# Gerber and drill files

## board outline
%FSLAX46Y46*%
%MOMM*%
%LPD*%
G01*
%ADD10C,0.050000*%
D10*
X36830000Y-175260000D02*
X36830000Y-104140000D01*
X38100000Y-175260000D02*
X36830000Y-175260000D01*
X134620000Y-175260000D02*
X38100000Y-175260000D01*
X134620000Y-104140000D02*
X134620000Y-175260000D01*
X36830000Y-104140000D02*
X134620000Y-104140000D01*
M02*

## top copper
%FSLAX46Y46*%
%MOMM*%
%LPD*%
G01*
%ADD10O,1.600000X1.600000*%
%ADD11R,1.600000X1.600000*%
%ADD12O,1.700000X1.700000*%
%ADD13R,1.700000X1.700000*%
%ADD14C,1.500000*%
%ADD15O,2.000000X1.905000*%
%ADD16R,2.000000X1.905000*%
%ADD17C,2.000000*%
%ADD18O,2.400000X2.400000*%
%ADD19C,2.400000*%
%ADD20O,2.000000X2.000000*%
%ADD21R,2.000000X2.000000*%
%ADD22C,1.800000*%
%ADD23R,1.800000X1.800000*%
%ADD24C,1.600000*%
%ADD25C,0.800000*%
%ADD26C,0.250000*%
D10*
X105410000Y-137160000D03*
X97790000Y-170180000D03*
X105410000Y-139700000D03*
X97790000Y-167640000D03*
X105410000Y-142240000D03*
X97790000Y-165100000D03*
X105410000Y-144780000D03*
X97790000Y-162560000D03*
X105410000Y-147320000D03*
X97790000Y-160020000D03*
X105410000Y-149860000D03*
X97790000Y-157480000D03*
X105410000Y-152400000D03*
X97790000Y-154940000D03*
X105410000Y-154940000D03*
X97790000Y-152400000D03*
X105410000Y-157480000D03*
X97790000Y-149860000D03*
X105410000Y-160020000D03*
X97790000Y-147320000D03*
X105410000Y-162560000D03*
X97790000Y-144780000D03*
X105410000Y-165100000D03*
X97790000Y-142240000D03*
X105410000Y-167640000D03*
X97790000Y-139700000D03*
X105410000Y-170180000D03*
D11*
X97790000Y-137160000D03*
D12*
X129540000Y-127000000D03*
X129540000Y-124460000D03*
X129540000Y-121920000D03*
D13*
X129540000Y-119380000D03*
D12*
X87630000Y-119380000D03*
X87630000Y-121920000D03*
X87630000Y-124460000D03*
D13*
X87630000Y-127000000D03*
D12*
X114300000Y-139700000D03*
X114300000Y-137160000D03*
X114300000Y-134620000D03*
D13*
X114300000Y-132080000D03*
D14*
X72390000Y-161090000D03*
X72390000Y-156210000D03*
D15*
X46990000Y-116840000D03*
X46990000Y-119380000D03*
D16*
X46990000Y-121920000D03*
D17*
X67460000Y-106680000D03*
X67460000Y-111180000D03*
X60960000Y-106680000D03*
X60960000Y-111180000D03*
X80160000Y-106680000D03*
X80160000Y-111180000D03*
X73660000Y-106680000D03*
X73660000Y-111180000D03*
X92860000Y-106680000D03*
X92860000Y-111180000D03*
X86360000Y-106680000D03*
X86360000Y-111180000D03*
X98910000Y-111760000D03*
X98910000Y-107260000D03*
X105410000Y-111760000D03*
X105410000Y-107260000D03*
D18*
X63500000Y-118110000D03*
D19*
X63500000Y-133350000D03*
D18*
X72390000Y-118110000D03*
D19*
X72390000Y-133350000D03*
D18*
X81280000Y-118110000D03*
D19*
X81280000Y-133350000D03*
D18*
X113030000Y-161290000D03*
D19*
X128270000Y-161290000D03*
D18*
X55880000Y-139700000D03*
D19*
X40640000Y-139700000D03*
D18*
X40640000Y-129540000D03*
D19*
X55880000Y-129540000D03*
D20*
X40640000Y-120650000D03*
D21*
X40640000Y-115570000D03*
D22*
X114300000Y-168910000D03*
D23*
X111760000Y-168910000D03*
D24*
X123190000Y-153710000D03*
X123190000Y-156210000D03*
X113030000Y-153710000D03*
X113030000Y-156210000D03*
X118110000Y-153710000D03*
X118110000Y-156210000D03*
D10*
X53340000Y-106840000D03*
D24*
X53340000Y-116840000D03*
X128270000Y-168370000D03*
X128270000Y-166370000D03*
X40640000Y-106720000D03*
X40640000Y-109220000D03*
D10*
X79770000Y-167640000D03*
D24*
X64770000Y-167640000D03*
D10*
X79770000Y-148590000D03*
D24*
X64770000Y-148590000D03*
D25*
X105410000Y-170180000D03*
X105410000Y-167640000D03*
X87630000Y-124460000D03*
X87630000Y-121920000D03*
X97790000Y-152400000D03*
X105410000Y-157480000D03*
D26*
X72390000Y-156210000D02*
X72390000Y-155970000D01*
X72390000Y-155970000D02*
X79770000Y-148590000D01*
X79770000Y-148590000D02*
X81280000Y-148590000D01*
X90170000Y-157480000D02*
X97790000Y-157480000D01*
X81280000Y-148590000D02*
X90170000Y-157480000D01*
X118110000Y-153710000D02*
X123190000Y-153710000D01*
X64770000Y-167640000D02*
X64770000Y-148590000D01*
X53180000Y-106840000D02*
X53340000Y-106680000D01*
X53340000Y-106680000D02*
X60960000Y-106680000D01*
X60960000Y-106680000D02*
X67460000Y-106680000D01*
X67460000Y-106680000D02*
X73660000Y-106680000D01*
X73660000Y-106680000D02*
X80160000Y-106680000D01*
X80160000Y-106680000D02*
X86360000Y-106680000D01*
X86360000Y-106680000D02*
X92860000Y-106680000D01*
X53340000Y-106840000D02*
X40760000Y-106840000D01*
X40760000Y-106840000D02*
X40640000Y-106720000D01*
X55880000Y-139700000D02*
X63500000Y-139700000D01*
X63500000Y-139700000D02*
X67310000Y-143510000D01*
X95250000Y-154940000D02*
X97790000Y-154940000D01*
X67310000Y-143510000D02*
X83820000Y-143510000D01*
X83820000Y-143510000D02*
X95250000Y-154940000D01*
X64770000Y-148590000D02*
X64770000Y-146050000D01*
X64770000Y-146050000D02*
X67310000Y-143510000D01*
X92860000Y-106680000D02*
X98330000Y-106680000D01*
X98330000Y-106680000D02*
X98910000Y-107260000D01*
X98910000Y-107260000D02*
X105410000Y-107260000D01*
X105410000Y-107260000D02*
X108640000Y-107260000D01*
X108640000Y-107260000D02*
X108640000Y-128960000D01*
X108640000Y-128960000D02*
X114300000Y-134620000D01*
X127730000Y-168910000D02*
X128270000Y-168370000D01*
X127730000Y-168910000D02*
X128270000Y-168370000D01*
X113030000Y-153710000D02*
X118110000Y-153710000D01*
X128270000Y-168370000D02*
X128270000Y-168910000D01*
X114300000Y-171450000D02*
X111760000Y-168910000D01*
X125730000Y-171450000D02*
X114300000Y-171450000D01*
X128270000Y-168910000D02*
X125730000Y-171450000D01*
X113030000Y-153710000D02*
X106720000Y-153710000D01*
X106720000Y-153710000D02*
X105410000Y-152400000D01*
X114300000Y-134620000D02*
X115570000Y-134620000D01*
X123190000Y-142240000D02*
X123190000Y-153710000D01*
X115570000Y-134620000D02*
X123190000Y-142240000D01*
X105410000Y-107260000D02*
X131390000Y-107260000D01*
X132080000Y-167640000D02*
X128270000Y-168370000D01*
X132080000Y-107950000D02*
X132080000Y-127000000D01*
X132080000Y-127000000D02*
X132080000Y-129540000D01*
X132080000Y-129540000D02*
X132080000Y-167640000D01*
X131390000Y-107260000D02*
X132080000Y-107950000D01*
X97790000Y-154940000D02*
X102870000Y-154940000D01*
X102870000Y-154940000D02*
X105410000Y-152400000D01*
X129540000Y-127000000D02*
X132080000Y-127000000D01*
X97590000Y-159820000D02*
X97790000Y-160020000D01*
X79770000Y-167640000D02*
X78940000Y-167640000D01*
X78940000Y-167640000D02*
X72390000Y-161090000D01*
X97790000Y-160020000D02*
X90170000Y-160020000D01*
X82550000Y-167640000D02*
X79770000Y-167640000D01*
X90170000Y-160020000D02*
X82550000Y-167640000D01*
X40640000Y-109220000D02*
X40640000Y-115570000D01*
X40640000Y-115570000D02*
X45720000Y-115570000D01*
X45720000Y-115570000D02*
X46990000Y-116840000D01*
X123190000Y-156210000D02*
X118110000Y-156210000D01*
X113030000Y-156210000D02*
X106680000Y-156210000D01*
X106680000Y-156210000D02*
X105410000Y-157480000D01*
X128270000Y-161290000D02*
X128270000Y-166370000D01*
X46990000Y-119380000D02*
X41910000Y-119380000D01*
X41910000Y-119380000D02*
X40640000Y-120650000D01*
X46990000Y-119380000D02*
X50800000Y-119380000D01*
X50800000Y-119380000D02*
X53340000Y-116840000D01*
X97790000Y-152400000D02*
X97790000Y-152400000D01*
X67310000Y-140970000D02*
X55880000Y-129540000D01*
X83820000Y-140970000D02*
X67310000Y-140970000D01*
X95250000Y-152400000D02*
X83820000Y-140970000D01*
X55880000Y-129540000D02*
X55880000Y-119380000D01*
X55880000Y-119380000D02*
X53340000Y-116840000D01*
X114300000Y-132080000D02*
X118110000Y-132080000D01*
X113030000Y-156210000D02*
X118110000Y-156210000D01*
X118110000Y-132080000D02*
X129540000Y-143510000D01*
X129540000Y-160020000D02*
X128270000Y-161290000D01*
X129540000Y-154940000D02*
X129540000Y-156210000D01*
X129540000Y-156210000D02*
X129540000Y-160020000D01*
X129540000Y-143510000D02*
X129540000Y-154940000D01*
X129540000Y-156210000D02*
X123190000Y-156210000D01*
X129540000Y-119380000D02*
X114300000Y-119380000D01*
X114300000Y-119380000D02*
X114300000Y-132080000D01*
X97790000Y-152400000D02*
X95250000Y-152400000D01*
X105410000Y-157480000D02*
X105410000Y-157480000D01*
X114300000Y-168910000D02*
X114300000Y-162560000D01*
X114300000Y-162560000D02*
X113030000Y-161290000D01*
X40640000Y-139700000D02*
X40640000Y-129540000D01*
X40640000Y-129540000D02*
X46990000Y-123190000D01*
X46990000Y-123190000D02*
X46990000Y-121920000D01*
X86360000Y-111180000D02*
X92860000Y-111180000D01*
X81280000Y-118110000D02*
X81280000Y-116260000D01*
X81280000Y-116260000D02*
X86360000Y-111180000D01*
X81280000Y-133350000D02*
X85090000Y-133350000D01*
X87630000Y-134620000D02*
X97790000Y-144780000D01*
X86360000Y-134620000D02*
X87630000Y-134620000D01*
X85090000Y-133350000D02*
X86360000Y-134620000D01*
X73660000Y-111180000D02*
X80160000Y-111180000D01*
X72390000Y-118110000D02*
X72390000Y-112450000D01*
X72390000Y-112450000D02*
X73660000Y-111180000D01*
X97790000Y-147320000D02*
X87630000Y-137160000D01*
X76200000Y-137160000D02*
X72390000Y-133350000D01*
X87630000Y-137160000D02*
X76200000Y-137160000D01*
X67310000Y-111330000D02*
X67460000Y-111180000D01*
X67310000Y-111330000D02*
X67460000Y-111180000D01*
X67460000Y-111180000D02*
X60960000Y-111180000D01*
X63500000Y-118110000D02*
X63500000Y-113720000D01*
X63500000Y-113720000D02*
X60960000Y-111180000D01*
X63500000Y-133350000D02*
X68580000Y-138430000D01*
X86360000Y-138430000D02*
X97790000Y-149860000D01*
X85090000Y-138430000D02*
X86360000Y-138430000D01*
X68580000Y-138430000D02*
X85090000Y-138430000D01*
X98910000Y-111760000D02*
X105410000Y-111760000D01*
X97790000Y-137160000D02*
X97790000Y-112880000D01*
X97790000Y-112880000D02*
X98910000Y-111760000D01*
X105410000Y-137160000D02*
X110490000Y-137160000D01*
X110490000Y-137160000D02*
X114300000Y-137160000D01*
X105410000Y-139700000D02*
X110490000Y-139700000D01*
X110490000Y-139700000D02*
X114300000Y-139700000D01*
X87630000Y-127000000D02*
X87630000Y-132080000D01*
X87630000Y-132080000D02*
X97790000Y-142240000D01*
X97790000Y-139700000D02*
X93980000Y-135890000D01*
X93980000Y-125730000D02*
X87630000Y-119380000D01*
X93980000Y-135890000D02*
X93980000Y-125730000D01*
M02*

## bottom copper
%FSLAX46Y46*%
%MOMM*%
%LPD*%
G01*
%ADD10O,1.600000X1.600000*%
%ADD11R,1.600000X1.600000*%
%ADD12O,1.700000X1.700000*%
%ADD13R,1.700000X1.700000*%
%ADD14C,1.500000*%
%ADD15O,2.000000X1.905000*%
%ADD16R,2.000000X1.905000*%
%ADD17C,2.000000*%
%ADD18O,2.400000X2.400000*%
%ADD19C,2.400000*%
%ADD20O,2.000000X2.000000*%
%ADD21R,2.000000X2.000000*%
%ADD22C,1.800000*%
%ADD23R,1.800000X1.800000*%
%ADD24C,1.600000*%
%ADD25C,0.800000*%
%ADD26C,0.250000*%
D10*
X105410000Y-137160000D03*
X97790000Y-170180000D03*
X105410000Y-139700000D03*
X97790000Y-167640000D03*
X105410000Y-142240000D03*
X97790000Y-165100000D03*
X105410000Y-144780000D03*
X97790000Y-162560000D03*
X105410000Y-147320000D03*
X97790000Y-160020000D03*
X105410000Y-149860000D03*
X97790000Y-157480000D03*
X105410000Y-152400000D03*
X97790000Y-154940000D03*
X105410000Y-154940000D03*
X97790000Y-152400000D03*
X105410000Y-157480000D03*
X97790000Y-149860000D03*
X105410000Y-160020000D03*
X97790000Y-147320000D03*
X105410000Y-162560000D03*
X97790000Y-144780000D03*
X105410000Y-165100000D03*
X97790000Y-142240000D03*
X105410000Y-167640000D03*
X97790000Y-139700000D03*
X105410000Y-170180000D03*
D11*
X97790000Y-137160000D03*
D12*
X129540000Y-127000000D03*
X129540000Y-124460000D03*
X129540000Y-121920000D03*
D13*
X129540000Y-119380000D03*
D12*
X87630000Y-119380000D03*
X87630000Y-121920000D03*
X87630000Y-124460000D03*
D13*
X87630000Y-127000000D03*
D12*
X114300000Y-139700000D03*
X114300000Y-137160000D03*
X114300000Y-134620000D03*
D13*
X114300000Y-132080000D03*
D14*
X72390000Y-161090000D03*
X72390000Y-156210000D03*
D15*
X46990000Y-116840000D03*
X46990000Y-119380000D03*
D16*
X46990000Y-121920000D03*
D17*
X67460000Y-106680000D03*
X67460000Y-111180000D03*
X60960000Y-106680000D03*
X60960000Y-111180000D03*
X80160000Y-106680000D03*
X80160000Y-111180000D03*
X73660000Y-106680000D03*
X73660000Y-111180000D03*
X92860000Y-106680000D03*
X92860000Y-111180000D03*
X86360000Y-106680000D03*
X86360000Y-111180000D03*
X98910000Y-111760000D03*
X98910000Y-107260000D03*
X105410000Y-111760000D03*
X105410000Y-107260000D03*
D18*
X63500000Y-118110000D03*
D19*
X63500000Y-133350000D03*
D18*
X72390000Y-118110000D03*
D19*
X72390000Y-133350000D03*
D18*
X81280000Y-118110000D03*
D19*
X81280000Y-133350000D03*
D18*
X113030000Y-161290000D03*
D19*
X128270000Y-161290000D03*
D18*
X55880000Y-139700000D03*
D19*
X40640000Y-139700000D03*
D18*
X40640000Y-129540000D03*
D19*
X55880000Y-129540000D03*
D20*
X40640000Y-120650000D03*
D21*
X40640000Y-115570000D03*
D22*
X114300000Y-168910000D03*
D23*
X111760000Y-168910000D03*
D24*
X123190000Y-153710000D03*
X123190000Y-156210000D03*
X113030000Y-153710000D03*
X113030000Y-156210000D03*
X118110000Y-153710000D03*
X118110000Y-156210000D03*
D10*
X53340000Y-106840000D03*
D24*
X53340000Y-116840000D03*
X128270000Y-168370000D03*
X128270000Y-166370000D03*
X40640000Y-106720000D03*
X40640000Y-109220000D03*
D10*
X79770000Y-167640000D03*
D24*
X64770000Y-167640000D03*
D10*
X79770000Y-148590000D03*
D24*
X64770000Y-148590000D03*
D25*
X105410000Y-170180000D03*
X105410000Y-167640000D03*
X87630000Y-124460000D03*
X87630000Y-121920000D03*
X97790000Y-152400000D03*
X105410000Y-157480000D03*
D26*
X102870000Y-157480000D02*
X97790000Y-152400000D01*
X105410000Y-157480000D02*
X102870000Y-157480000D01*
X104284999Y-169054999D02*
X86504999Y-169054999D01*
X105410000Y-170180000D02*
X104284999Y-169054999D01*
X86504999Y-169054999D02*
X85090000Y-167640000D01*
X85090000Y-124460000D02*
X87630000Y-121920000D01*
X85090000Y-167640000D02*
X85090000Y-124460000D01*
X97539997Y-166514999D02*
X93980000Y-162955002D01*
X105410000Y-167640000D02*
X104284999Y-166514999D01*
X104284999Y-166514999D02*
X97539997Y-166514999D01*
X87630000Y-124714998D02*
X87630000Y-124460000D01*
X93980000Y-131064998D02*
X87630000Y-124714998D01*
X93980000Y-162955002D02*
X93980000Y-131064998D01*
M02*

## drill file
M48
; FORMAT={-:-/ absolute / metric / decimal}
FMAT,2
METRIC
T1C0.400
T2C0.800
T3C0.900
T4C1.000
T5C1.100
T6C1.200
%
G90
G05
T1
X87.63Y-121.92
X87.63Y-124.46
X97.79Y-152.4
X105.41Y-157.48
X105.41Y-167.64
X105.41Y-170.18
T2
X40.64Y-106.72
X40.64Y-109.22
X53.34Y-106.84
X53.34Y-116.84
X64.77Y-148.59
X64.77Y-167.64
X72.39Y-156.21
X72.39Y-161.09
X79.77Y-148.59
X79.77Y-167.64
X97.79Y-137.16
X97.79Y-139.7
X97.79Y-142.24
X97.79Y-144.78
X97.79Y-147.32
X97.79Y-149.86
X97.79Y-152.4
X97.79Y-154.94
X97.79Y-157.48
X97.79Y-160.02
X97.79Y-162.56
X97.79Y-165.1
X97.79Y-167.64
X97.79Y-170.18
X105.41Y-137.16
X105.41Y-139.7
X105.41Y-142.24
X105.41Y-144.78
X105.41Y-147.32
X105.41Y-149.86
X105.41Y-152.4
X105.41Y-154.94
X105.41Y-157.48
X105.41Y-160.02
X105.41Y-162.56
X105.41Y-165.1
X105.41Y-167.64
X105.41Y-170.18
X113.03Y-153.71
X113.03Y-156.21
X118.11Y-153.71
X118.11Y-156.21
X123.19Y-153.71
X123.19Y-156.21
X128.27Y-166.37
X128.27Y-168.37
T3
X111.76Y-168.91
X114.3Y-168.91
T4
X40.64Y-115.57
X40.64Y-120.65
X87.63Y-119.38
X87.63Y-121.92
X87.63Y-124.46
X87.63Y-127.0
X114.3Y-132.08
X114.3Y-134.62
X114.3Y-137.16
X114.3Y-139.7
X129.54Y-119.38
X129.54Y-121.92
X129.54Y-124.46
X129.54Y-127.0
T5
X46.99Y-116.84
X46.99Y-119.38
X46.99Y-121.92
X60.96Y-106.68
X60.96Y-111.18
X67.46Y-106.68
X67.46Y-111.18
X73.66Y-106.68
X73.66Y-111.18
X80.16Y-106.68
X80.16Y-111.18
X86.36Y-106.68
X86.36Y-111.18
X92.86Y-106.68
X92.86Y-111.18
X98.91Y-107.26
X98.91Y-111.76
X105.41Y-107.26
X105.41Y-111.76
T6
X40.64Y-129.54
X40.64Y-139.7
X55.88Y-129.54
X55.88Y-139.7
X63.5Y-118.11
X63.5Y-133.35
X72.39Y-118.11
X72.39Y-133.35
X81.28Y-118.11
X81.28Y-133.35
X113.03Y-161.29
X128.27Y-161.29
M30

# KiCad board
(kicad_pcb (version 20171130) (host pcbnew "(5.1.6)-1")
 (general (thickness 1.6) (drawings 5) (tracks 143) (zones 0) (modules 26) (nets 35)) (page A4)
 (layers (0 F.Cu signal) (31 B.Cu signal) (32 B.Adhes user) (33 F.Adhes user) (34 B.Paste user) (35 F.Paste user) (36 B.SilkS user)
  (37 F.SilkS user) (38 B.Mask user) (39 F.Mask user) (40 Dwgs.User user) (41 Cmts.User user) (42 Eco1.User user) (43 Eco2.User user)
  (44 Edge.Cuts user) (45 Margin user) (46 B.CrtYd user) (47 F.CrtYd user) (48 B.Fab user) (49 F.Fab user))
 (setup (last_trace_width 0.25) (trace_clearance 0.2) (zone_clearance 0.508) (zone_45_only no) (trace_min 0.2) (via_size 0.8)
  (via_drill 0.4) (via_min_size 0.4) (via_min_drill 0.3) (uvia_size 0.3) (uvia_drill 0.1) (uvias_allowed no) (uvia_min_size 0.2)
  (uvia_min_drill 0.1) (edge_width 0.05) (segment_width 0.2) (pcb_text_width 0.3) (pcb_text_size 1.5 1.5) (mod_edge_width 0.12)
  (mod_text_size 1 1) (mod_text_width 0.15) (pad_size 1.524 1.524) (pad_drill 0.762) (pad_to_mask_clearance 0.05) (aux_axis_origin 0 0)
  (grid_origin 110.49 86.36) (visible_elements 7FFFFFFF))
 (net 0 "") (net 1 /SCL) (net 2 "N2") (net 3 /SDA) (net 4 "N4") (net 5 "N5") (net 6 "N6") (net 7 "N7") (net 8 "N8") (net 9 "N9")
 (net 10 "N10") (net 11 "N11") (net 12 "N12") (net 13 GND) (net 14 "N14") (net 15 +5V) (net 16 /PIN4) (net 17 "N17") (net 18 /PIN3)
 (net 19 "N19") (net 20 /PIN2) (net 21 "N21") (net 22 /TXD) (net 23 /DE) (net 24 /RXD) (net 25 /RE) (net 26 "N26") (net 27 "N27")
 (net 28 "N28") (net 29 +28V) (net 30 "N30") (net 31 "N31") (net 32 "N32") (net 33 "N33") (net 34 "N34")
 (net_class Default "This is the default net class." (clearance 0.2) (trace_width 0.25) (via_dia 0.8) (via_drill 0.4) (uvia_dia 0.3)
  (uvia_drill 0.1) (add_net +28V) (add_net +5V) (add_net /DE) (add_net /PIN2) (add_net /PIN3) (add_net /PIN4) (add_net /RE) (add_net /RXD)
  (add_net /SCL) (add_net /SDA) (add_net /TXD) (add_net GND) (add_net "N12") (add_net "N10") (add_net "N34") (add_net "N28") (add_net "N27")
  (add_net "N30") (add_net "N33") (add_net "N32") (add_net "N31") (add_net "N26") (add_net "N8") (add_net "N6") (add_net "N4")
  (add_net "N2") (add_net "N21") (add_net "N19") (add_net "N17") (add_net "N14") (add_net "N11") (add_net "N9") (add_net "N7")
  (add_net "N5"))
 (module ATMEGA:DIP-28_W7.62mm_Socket (layer F.Cu) (at 97.79 137.16)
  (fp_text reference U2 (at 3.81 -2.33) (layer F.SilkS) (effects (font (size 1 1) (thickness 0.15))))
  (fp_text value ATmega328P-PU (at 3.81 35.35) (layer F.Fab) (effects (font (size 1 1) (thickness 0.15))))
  (pad 28 thru_hole oval (at 7.62 0) (size 1.6 1.6) (drill 0.8) (layers *.Cu *.Mask) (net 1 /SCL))
  (pad 14 thru_hole oval (at 0 33.02) (size 1.6 1.6) (drill 0.8) (layers *.Cu *.Mask) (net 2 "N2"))
  (pad 27 thru_hole oval (at 7.62 2.54) (size 1.6 1.6) (drill 0.8) (layers *.Cu *.Mask) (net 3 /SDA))
  (pad 13 thru_hole oval (at 0 30.48) (size 1.6 1.6) (drill 0.8) (layers *.Cu *.Mask) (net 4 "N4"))
  (pad 26 thru_hole oval (at 7.62 5.08) (size 1.6 1.6) (drill 0.8) (layers *.Cu *.Mask) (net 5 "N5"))
  (pad 12 thru_hole oval (at 0 27.94) (size 1.6 1.6) (drill 0.8) (layers *.Cu *.Mask) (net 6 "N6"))
  (pad 25 thru_hole oval (at 7.62 7.62) (size 1.6 1.6) (drill 0.8) (layers *.Cu *.Mask) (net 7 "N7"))
  (pad 11 thru_hole oval (at 0 25.4) (size 1.6 1.6) (drill 0.8) (layers *.Cu *.Mask) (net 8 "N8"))
  (pad 24 thru_hole oval (at 7.62 10.16) (size 1.6 1.6) (drill 0.8) (layers *.Cu *.Mask) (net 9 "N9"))
  (pad 10 thru_hole oval (at 0 22.86) (size 1.6 1.6) (drill 0.8) (layers *.Cu *.Mask) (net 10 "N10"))
  (pad 23 thru_hole oval (at 7.62 12.7) (size 1.6 1.6) (drill 0.8) (layers *.Cu *.Mask) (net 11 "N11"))
  (pad 9 thru_hole oval (at 0 20.32) (size 1.6 1.6) (drill 0.8) (layers *.Cu *.Mask) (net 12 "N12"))
  (pad 22 thru_hole oval (at 7.62 15.24) (size 1.6 1.6) (drill 0.8) (layers *.Cu *.Mask) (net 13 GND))
  (pad 8 thru_hole oval (at 0 17.78) (size 1.6 1.6) (drill 0.8) (layers *.Cu *.Mask) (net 13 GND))
  (pad 21 thru_hole oval (at 7.62 17.78) (size 1.6 1.6) (drill 0.8) (layers *.Cu *.Mask) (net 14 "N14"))
  (pad 7 thru_hole oval (at 0 15.24) (size 1.6 1.6) (drill 0.8) (layers *.Cu *.Mask) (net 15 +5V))
  (pad 20 thru_hole oval (at 7.62 20.32) (size 1.6 1.6) (drill 0.8) (layers *.Cu *.Mask) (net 15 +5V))
  (pad 6 thru_hole oval (at 0 12.7) (size 1.6 1.6) (drill 0.8) (layers *.Cu *.Mask) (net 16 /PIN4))
  (pad 19 thru_hole oval (at 7.62 22.86) (size 1.6 1.6) (drill 0.8) (layers *.Cu *.Mask) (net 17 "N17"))
  (pad 5 thru_hole oval (at 0 10.16) (size 1.6 1.6) (drill 0.8) (layers *.Cu *.Mask) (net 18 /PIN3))
  (pad 18 thru_hole oval (at 7.62 25.4) (size 1.6 1.6) (drill 0.8) (layers *.Cu *.Mask) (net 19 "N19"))
  (pad 4 thru_hole oval (at 0 7.62) (size 1.6 1.6) (drill 0.8) (layers *.Cu *.Mask) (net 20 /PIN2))
  (pad 17 thru_hole oval (at 7.62 27.94) (size 1.6 1.6) (drill 0.8) (layers *.Cu *.Mask) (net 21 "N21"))
  (pad 3 thru_hole oval (at 0 5.08) (size 1.6 1.6) (drill 0.8) (layers *.Cu *.Mask) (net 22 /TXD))
  (pad 16 thru_hole oval (at 7.62 30.48) (size 1.6 1.6) (drill 0.8) (layers *.Cu *.Mask) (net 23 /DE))
  (pad 2 thru_hole oval (at 0 2.54) (size 1.6 1.6) (drill 0.8) (layers *.Cu *.Mask) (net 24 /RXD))
  (pad 15 thru_hole oval (at 7.62 33.02) (size 1.6 1.6) (drill 0.8) (layers *.Cu *.Mask) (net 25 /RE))
  (pad 1 thru_hole rect (at 0 0) (size 1.6 1.6) (drill 0.8) (layers *.Cu *.Mask) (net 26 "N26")))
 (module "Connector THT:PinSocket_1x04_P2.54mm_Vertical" (layer F.Cu) (at 129.54 119.38)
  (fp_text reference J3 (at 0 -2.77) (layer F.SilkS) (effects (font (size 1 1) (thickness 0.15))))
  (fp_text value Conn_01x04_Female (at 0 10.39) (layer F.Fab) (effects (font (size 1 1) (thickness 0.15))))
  (pad 4 thru_hole oval (at 0 7.62) (size 1.7 1.7) (drill 1) (layers *.Cu *.Mask) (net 13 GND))
  (pad 3 thru_hole oval (at 0 5.08) (size 1.7 1.7) (drill 1) (layers *.Cu *.Mask) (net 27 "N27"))
  (pad 2 thru_hole oval (at 0 2.54) (size 1.7 1.7) (drill 1) (layers *.Cu *.Mask) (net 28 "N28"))
  (pad 1 thru_hole rect (at 0 0) (size 1.7 1.7) (drill 1) (layers *.Cu *.Mask) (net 15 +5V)))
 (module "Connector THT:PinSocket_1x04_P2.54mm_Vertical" (layer F.Cu) (at 87.63 127 180)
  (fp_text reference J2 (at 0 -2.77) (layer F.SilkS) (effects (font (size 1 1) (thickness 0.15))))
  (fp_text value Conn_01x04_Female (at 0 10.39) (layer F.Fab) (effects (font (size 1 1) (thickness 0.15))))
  (pad 4 thru_hole oval (at 0 7.62 180) (size 1.7 1.7) (drill 1) (layers *.Cu *.Mask) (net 24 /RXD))
  (pad 3 thru_hole oval (at 0 5.08 180) (size 1.7 1.7) (drill 1) (layers *.Cu *.Mask) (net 25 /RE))
  (pad 2 thru_hole oval (at 0 2.54 180) (size 1.7 1.7) (drill 1) (layers *.Cu *.Mask) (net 23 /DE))
  (pad 1 thru_hole rect (at 0 0 180) (size 1.7 1.7) (drill 1) (layers *.Cu *.Mask) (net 22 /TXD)))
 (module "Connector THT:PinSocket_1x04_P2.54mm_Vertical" (layer F.Cu) (at 114.3 132.08)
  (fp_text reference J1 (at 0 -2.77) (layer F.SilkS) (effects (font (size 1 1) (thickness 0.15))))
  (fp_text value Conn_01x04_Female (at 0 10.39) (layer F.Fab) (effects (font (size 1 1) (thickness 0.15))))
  (pad 4 thru_hole oval (at 0 7.62) (size 1.7 1.7) (drill 1) (layers *.Cu *.Mask) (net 3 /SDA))
  (pad 3 thru_hole oval (at 0 5.08) (size 1.7 1.7) (drill 1) (layers *.Cu *.Mask) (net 1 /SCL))
  (pad 2 thru_hole oval (at 0 2.54) (size 1.7 1.7) (drill 1) (layers *.Cu *.Mask) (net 13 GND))
  (pad 1 thru_hole rect (at 0 0) (size 1.7 1.7) (drill 1) (layers *.Cu *.Mask) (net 15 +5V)))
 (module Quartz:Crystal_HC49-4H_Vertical (layer F.Cu) (at 72.39 156.21 270)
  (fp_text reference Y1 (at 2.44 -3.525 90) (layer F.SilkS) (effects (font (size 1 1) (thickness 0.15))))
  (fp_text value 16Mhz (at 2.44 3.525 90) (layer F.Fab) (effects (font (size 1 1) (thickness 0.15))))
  (pad 2 thru_hole circle (at 4.88 0 270) (size 1.5 1.5) (drill 0.8) (layers *.Cu *.Mask) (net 10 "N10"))
  (pad 1 thru_hole circle (at 0 0 270) (size 1.5 1.5) (drill 0.8) (layers *.Cu *.Mask) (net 12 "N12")))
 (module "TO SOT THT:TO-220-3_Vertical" (layer F.Cu) (at 46.99 121.92 90)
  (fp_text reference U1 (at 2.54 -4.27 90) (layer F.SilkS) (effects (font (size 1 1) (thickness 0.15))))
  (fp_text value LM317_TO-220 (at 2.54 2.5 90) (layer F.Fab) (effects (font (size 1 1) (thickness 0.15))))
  (pad 3 thru_hole oval (at 5.08 0 90) (size 1.905 2) (drill 1.1) (layers *.Cu *.Mask) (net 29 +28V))
  (pad 2 thru_hole oval (at 2.54 0 90) (size 1.905 2) (drill 1.1) (layers *.Cu *.Mask) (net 15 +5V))
  (pad 1 thru_hole rect (at 0 0 90) (size 1.905 2) (drill 1.1) (layers *.Cu *.Mask) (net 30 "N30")))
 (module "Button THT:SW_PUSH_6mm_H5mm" (layer F.Cu) (at 60.96 106.68)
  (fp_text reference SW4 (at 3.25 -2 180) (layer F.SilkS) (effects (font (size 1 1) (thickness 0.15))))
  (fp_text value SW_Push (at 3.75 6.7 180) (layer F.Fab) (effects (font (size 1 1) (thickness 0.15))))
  (pad 1 thru_hole circle (at 6.5 0 90) (size 2 2) (drill 1.1) (layers *.Cu *.Mask) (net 13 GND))
  (pad 2 thru_hole circle (at 6.5 4.5 90) (size 2 2) (drill 1.1) (layers *.Cu *.Mask) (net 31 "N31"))
  (pad 1 thru_hole circle (at 0 0 90) (size 2 2) (drill 1.1) (layers *.Cu *.Mask) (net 13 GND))
  (pad 2 thru_hole circle (at 0 4.5 90) (size 2 2) (drill 1.1) (layers *.Cu *.Mask) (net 31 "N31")))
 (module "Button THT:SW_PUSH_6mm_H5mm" (layer F.Cu) (at 73.66 106.68)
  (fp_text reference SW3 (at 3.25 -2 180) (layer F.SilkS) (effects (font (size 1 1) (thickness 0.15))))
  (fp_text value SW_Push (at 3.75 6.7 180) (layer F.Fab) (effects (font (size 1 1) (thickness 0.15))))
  (pad 1 thru_hole circle (at 6.5 0 90) (size 2 2) (drill 1.1) (layers *.Cu *.Mask) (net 13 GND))
  (pad 2 thru_hole circle (at 6.5 4.5 90) (size 2 2) (drill 1.1) (layers *.Cu *.Mask) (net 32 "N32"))
  (pad 1 thru_hole circle (at 0 0 90) (size 2 2) (drill 1.1) (layers *.Cu *.Mask) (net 13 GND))
  (pad 2 thru_hole circle (at 0 4.5 90) (size 2 2) (drill 1.1) (layers *.Cu *.Mask) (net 32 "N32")))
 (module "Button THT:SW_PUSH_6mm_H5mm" (layer F.Cu) (at 86.36 106.68)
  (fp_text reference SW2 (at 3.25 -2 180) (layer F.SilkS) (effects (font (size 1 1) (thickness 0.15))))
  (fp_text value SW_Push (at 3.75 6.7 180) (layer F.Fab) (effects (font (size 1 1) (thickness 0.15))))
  (pad 1 thru_hole circle (at 6.5 0 90) (size 2 2) (drill 1.1) (layers *.Cu *.Mask) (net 13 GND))
  (pad 2 thru_hole circle (at 6.5 4.5 90) (size 2 2) (drill 1.1) (layers *.Cu *.Mask) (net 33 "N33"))
  (pad 1 thru_hole circle (at 0 0 90) (size 2 2) (drill 1.1) (layers *.Cu *.Mask) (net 13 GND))
  (pad 2 thru_hole circle (at 0 4.5 90) (size 2 2) (drill 1.1) (layers *.Cu *.Mask) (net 33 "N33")))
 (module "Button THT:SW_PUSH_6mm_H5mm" (layer F.Cu) (at 105.41 111.76 180)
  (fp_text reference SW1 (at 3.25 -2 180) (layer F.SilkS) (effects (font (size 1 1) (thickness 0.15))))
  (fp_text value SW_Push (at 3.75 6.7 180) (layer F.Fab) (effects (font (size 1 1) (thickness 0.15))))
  (pad 1 thru_hole circle (at 6.5 0 270) (size 2 2) (drill 1.1) (layers *.Cu *.Mask) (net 26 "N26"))
  (pad 2 thru_hole circle (at 6.5 4.5 270) (size 2 2) (drill 1.1) (layers *.Cu *.Mask) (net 13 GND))
  (pad 1 thru_hole circle (at 0 0 270) (size 2 2) (drill 1.1) (layers *.Cu *.Mask) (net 26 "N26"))
  (pad 2 thru_hole circle (at 0 4.5 270) (size 2 2) (drill 1.1) (layers *.Cu *.Mask) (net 13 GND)))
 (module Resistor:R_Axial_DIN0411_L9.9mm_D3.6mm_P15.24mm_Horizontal (layer F.Cu) (at 63.5 133.35 90)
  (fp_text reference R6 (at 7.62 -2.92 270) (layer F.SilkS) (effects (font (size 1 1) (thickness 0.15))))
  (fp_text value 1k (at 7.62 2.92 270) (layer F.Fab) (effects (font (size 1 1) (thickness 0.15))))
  (pad 2 thru_hole oval (at 15.24 0 90) (size 2.4 2.4) (drill 1.2) (layers *.Cu *.Mask) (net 31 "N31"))
  (pad 1 thru_hole circle (at 0 0 90) (size 2.4 2.4) (drill 1.2) (layers *.Cu *.Mask) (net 16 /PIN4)))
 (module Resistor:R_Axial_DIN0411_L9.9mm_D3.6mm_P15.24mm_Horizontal (layer F.Cu) (at 72.39 133.35 90)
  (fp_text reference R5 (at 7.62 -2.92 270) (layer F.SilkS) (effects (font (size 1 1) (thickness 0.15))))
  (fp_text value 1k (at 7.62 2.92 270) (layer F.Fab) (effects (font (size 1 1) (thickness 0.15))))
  (pad 2 thru_hole oval (at 15.24 0 90) (size 2.4 2.4) (drill 1.2) (layers *.Cu *.Mask) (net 32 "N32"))
  (pad 1 thru_hole circle (at 0 0 90) (size 2.4 2.4) (drill 1.2) (layers *.Cu *.Mask) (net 18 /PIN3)))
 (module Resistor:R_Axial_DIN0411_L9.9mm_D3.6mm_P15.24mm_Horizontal (layer F.Cu) (at 81.28 133.35 90)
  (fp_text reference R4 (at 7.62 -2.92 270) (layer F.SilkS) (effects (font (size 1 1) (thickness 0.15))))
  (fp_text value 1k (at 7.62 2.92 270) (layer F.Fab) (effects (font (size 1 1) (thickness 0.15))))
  (pad 2 thru_hole oval (at 15.24 0 90) (size 2.4 2.4) (drill 1.2) (layers *.Cu *.Mask) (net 33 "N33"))
  (pad 1 thru_hole circle (at 0 0 90) (size 2.4 2.4) (drill 1.2) (layers *.Cu *.Mask) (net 20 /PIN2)))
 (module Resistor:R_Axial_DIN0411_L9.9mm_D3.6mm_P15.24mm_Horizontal (layer F.Cu) (at 128.27 161.29 180)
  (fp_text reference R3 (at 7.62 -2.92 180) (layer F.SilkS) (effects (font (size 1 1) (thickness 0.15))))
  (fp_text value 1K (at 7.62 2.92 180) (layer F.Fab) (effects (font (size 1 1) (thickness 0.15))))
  (pad 2 thru_hole oval (at 15.24 0 180) (size 2.4 2.4) (drill 1.2) (layers *.Cu *.Mask) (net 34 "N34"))
  (pad 1 thru_hole circle (at 0 0 180) (size 2.4 2.4) (drill 1.2) (layers *.Cu *.Mask) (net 15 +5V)))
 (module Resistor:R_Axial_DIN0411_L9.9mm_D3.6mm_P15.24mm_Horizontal (layer F.Cu) (at 40.64 139.7)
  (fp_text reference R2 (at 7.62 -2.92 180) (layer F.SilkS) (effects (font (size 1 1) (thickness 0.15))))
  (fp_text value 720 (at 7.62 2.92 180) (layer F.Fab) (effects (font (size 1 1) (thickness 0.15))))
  (pad 2 thru_hole oval (at 15.24 0) (size 2.4 2.4) (drill 1.2) (layers *.Cu *.Mask) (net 13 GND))
  (pad 1 thru_hole circle (at 0 0) (size 2.4 2.4) (drill 1.2) (layers *.Cu *.Mask) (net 30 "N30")))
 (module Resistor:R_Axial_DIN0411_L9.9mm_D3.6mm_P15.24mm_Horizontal (layer F.Cu) (at 55.88 129.54 180)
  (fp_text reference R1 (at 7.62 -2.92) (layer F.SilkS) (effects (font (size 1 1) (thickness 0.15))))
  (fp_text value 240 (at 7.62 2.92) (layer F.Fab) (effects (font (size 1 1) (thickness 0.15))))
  (pad 2 thru_hole oval (at 15.24 0 180) (size 2.4 2.4) (drill 1.2) (layers *.Cu *.Mask) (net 30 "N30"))
  (pad 1 thru_hole circle (at 0 0 180) (size 2.4 2.4) (drill 1.2) (layers *.Cu *.Mask) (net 15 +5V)))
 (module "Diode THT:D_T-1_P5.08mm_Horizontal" (layer F.Cu) (at 40.64 115.57 270)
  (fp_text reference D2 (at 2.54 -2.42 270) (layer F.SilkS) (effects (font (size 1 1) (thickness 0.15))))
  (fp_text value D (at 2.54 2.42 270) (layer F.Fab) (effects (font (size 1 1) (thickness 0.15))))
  (pad 2 thru_hole oval (at 5.08 0 270) (size 2 2) (drill 1) (layers *.Cu *.Mask) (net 15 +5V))
  (pad 1 thru_hole rect (at 0 0 270) (size 2 2) (drill 1) (layers *.Cu *.Mask) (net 29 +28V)))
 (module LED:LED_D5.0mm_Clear (layer F.Cu) (at 111.76 168.91)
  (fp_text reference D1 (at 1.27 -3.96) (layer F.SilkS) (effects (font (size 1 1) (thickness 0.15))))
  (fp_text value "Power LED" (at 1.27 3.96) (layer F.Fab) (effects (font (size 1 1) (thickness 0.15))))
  (pad 2 thru_hole circle (at 2.54 0) (size 1.8 1.8) (drill 0.9) (layers *.Cu *.Mask) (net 34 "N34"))
  (pad 1 thru_hole rect (at 0 0) (size 1.8 1.8) (drill 0.9) (layers *.Cu *.Mask) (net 13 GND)))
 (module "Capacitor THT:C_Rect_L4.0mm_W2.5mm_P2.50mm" (layer F.Cu) (at 123.19 156.21 90)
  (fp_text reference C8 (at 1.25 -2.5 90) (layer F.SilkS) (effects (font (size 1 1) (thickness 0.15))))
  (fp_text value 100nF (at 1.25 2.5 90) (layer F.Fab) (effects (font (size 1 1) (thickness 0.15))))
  (pad 2 thru_hole circle (at 2.5 0 90) (size 1.6 1.6) (drill 0.8) (layers *.Cu *.Mask) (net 13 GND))
  (pad 1 thru_hole circle (at 0 0 90) (size 1.6 1.6) (drill 0.8) (layers *.Cu *.Mask) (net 15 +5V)))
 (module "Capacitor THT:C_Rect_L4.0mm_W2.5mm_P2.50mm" (layer F.Cu) (at 113.03 156.21 90)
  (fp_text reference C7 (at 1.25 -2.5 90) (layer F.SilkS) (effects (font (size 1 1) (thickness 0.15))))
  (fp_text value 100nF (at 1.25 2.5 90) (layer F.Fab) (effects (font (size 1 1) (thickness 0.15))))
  (pad 2 thru_hole circle (at 2.5 0 90) (size 1.6 1.6) (drill 0.8) (layers *.Cu *.Mask) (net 13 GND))
  (pad 1 thru_hole circle (at 0 0 90) (size 1.6 1.6) (drill 0.8) (layers *.Cu *.Mask) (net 15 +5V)))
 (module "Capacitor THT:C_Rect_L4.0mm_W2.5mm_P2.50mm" (layer F.Cu) (at 118.11 156.21 90)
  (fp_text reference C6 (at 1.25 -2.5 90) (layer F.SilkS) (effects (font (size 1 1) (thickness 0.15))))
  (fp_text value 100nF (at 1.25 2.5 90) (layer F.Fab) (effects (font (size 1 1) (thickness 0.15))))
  (pad 2 thru_hole circle (at 2.5 0 90) (size 1.6 1.6) (drill 0.8) (layers *.Cu *.Mask) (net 13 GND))
  (pad 1 thru_hole circle (at 0 0 90) (size 1.6 1.6) (drill 0.8) (layers *.Cu *.Mask) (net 15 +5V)))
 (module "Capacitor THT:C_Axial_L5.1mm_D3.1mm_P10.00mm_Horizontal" (layer F.Cu) (at 53.34 116.84 90)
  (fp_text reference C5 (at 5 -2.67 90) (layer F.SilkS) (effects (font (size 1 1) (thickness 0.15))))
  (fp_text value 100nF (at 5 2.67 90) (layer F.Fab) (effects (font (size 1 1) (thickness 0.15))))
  (pad 2 thru_hole oval (at 10 0 90) (size 1.6 1.6) (drill 0.8) (layers *.Cu *.Mask) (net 13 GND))
  (pad 1 thru_hole circle (at 0 0 90) (size 1.6 1.6) (drill 0.8) (layers *.Cu *.Mask) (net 15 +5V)))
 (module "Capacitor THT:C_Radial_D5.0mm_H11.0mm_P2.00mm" (layer F.Cu) (at 128.27 166.37 270)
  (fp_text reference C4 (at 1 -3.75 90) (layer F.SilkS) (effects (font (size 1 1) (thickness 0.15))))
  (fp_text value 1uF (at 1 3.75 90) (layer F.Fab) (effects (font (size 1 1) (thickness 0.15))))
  (pad 2 thru_hole circle (at 2 0 270) (size 1.6 1.6) (drill 0.8) (layers *.Cu *.Mask) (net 13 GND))
  (pad 1 thru_hole circle (at 0 0 270) (size 1.6 1.6) (drill 0.8) (layers *.Cu *.Mask) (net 15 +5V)))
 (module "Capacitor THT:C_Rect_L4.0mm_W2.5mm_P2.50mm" (layer F.Cu) (at 40.64 109.22 90)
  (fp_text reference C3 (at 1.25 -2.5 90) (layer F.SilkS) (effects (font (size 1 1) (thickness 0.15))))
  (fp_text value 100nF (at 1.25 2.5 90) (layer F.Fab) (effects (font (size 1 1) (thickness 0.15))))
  (pad 2 thru_hole circle (at 2.5 0 90) (size 1.6 1.6) (drill 0.8) (layers *.Cu *.Mask) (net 13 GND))
  (pad 1 thru_hole circle (at 0 0 90) (size 1.6 1.6) (drill 0.8) (layers *.Cu *.Mask) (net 29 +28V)))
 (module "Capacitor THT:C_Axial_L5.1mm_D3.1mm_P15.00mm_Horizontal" (layer F.Cu) (at 64.77 167.64)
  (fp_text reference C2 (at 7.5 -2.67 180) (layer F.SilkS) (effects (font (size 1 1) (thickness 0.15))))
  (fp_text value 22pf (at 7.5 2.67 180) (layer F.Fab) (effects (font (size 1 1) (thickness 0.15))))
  (pad 2 thru_hole oval (at 15 0) (size 1.6 1.6) (drill 0.8) (layers *.Cu *.Mask) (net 10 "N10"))
  (pad 1 thru_hole circle (at 0 0) (size 1.6 1.6) (drill 0.8) (layers *.Cu *.Mask) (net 13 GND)))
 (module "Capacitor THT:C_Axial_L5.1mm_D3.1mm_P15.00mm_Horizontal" (layer F.Cu) (at 64.77 148.59)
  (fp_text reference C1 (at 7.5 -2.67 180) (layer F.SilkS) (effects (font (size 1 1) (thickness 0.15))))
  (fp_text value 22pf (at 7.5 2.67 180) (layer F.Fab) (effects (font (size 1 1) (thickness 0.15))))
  (pad 2 thru_hole oval (at 15 0) (size 1.6 1.6) (drill 0.8) (layers *.Cu *.Mask) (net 12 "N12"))
  (pad 1 thru_hole circle (at 0 0) (size 1.6 1.6) (drill 0.8) (layers *.Cu *.Mask) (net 13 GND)))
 (gr_line (start 36.83 175.26) (end 36.83 104.14) (angle 90) (layer Edge.Cuts) (width 0.05))
 (gr_line (start 38.1 175.26) (end 36.83 175.26) (angle 90) (layer Edge.Cuts) (width 0.05))
 (gr_line (start 134.62 175.26) (end 38.1 175.26) (angle 90) (layer Edge.Cuts) (width 0.05))
 (gr_line (start 134.62 104.14) (end 134.62 175.26) (angle 90) (layer Edge.Cuts) (width 0.05))
 (gr_line (start 36.83 104.14) (end 134.62 104.14) (angle 90) (layer Edge.Cuts) (width 0.05))
 (via (at 105.41 170.18) (size 0.8) (drill 0.4) (layers F.Cu B.Cu) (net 25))
 (via (at 105.41 167.64) (size 0.8) (drill 0.4) (layers F.Cu B.Cu) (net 23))
 (via (at 87.63 124.46) (size 0.8) (drill 0.4) (layers F.Cu B.Cu) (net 23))
 (via (at 87.63 121.92) (size 0.8) (drill 0.4) (layers F.Cu B.Cu) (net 25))
 (segment (start 72.39 156.21) (end 72.39 155.97) (width 0.25) (layer F.Cu) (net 12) (status C00000))
 (segment (start 72.39 155.97) (end 79.77 148.59) (width 0.25) (layer F.Cu) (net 12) (status C00000))
 (segment (start 79.77 148.59) (end 81.28 148.59) (width 0.25) (layer F.Cu) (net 12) (status 400000))
 (segment (start 90.17 157.48) (end 97.79 157.48) (width 0.25) (layer F.Cu) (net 12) (status 800000))
 (segment (start 81.28 148.59) (end 90.17 157.48) (width 0.25) (layer F.Cu) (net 12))
 (segment (start 118.11 153.71) (end 123.19 153.71) (width 0.25) (layer F.Cu) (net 13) (status C00000))
 (segment (start 64.77 167.64) (end 64.77 148.59) (width 0.25) (layer F.Cu) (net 13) (status C00000))
 (segment (start 53.18 106.84) (end 53.34 106.68) (width 0.25) (layer F.Cu) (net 13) (status C00000))
 (segment (start 53.34 106.68) (end 60.96 106.68) (width 0.25) (layer F.Cu) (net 13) (status C00000))
 (segment (start 60.96 106.68) (end 67.46 106.68) (width 0.25) (layer F.Cu) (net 13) (status C00000))
 (segment (start 67.46 106.68) (end 73.66 106.68) (width 0.25) (layer F.Cu) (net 13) (status C00000))
 (segment (start 73.66 106.68) (end 80.16 106.68) (width 0.25) (layer F.Cu) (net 13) (status C00000))
 (segment (start 80.16 106.68) (end 86.36 106.68) (width 0.25) (layer F.Cu) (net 13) (status C00000))
 (segment (start 86.36 106.68) (end 92.86 106.68) (width 0.25) (layer F.Cu) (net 13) (status C00000))
 (segment (start 53.34 106.84) (end 40.76 106.84) (width 0.25) (layer F.Cu) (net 13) (status C00000))
 (segment (start 40.76 106.84) (end 40.64 106.72) (width 0.25) (layer F.Cu) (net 13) (status C00000))
 (segment (start 55.88 139.7) (end 63.5 139.7) (width 0.25) (layer F.Cu) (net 13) (status 400000))
 (segment (start 63.5 139.7) (end 67.31 143.51) (width 0.25) (layer F.Cu) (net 13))
 (segment (start 95.25 154.94) (end 97.79 154.94) (width 0.25) (layer F.Cu) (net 13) (status 800000))
 (segment (start 67.31 143.51) (end 83.82 143.51) (width 0.25) (layer F.Cu) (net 13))
 (segment (start 83.82 143.51) (end 95.25 154.94) (width 0.25) (layer F.Cu) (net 13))
 (segment (start 64.77 148.59) (end 64.77 146.05) (width 0.25) (layer F.Cu) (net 13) (status 400000))
 (segment (start 64.77 146.05) (end 67.31 143.51) (width 0.25) (layer F.Cu) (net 13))
 (segment (start 92.86 106.68) (end 98.33 106.68) (width 0.25) (layer F.Cu) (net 13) (status C00000))
 (segment (start 98.33 106.68) (end 98.91 107.26) (width 0.25) (layer F.Cu) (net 13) (status C00000))
 (segment (start 98.91 107.26) (end 105.41 107.26) (width 0.25) (layer F.Cu) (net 13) (status C00000))
 (segment (start 105.41 107.26) (end 108.64 107.26) (width 0.25) (layer F.Cu) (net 13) (status 400000))
 (segment (start 108.64 107.26) (end 108.64 128.96) (width 0.25) (layer F.Cu) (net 13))
 (segment (start 108.64 128.96) (end 114.3 134.62) (width 0.25) (layer F.Cu) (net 13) (status 800000))
 (segment (start 127.73 168.91) (end 128.27 168.37) (width 0.25) (layer F.Cu) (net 13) (status C00000))
 (segment (start 127.73 168.91) (end 128.27 168.37) (width 0.25) (layer F.Cu) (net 13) (status C00000))
 (segment (start 113.03 153.71) (end 118.11 153.71) (width 0.25) (layer F.Cu) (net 13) (status C00000))
 (segment (start 128.27 168.37) (end 128.27 168.91) (width 0.25) (layer F.Cu) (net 13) (status C00000))
 (segment (start 114.3 171.45) (end 111.76 168.91) (width 0.25) (layer F.Cu) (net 13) (status 800000))
 (segment (start 125.73 171.45) (end 114.3 171.45) (width 0.25) (layer F.Cu) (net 13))
 (segment (start 128.27 168.91) (end 125.73 171.45) (width 0.25) (layer F.Cu) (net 13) (status 400000))
 (segment (start 113.03 153.71) (end 106.72 153.71) (width 0.25) (layer F.Cu) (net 13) (status 400000))
 (segment (start 106.72 153.71) (end 105.41 152.4) (width 0.25) (layer F.Cu) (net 13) (status 800000))
 (segment (start 114.3 134.62) (end 115.57 134.62) (width 0.25) (layer F.Cu) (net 13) (status 400000))
 (segment (start 123.19 142.24) (end 123.19 153.71) (width 0.25) (layer F.Cu) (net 13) (status 800000))
 (segment (start 115.57 134.62) (end 123.19 142.24) (width 0.25) (layer F.Cu) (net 13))
 (segment (start 105.41 107.26) (end 131.39 107.26) (width 0.25) (layer F.Cu) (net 13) (status 400000))
 (segment (start 132.08 167.64) (end 128.27 168.37) (width 0.25) (layer F.Cu) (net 13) (status 800000))
 (segment (start 132.08 107.95) (end 132.08 127) (width 0.25) (layer F.Cu) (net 13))
 (segment (start 132.08 127) (end 132.08 129.54) (width 0.25) (layer F.Cu) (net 13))
 (segment (start 132.08 129.54) (end 132.08 167.64) (width 0.25) (layer F.Cu) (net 13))
 (segment (start 131.39 107.26) (end 132.08 107.95) (width 0.25) (layer F.Cu) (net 13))
 (segment (start 97.79 154.94) (end 102.87 154.94) (width 0.25) (layer F.Cu) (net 13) (status 400000))
 (segment (start 102.87 154.94) (end 105.41 152.4) (width 0.25) (layer F.Cu) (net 13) (status 800000))
 (segment (start 129.54 127) (end 132.08 127) (width 0.25) (layer F.Cu) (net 13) (status 400000))
 (segment (start 97.59 159.82) (end 97.79 160.02) (width 0.25) (layer F.Cu) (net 10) (status C00000))
 (segment (start 79.77 167.64) (end 78.94 167.64) (width 0.25) (layer F.Cu) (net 10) (status 400000))
 (segment (start 78.94 167.64) (end 72.39 161.09) (width 0.25) (layer F.Cu) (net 10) (status 800000))
 (segment (start 97.79 160.02) (end 90.17 160.02) (width 0.25) (layer F.Cu) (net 10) (status 400000))
 (segment (start 82.55 167.64) (end 79.77 167.64) (width 0.25) (layer F.Cu) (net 10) (status 800000))
 (segment (start 90.17 160.02) (end 82.55 167.64) (width 0.25) (layer F.Cu) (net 10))
 (segment (start 40.64 109.22) (end 40.64 115.57) (width 0.25) (layer F.Cu) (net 29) (status C00000))
 (segment (start 40.64 115.57) (end 45.72 115.57) (width 0.25) (layer F.Cu) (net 29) (status 400000))
 (segment (start 45.72 115.57) (end 46.99 116.84) (width 0.25) (layer F.Cu) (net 29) (status 800000))
 (segment (start 123.19 156.21) (end 118.11 156.21) (width 0.25) (layer F.Cu) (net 15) (status C00000))
 (segment (start 113.03 156.21) (end 106.68 156.21) (width 0.25) (layer F.Cu) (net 15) (status 400000))
 (segment (start 106.68 156.21) (end 105.41 157.48) (width 0.25) (layer F.Cu) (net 15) (status 800000))
 (segment (start 128.27 161.29) (end 128.27 166.37) (width 0.25) (layer F.Cu) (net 15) (status C00000))
 (segment (start 46.99 119.38) (end 41.91 119.38) (width 0.25) (layer F.Cu) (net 15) (status 400000))
 (segment (start 41.91 119.38) (end 40.64 120.65) (width 0.25) (layer F.Cu) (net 15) (status 800000))
 (segment (start 46.99 119.38) (end 50.8 119.38) (width 0.25) (layer F.Cu) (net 15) (status 400000))
 (segment (start 50.8 119.38) (end 53.34 116.84) (width 0.25) (layer F.Cu) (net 15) (status 800000))
 (segment (start 97.79 152.4) (end 97.79 152.4) (width 0.25) (layer F.Cu) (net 15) (status 400000))
 (segment (start 67.31 140.97) (end 55.88 129.54) (width 0.25) (layer F.Cu) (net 15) (status 800000))
 (segment (start 83.82 140.97) (end 67.31 140.97) (width 0.25) (layer F.Cu) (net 15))
 (segment (start 95.25 152.4) (end 83.82 140.97) (width 0.25) (layer F.Cu) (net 15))
 (segment (start 55.88 129.54) (end 55.88 119.38) (width 0.25) (layer F.Cu) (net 15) (status 400000))
 (segment (start 55.88 119.38) (end 53.34 116.84) (width 0.25) (layer F.Cu) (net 15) (status 800000))
 (segment (start 114.3 132.08) (end 118.11 132.08) (width 0.25) (layer F.Cu) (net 15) (status 400000))
 (segment (start 113.03 156.21) (end 118.11 156.21) (width 0.25) (layer F.Cu) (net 15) (status C00000))
 (segment (start 118.11 132.08) (end 129.54 143.51) (width 0.25) (layer F.Cu) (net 15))
 (segment (start 129.54 160.02) (end 128.27 161.29) (width 0.25) (layer F.Cu) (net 15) (status 800000))
 (segment (start 129.54 154.94) (end 129.54 156.21) (width 0.25) (layer F.Cu) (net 15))
 (segment (start 129.54 156.21) (end 129.54 160.02) (width 0.25) (layer F.Cu) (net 15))
 (segment (start 129.54 143.51) (end 129.54 154.94) (width 0.25) (layer F.Cu) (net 15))
 (segment (start 129.54 156.21) (end 123.19 156.21) (width 0.25) (layer F.Cu) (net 15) (status 800000))
 (segment (start 129.54 119.38) (end 114.3 119.38) (width 0.25) (layer F.Cu) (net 15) (status 400000))
 (segment (start 114.3 119.38) (end 114.3 132.08) (width 0.25) (layer F.Cu) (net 15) (status 800000))
 (segment (start 97.79 152.4) (end 95.25 152.4) (width 0.25) (layer F.Cu) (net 15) (status 400000))
 (via (at 97.79 152.4) (size 0.8) (drill 0.4) (layers F.Cu B.Cu) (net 15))
 (segment (start 105.41 157.48) (end 105.41 157.48) (width 0.25) (layer F.Cu) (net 15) (status 800000))
 (via (at 105.41 157.48) (size 0.8) (drill 0.4) (layers F.Cu B.Cu) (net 15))
 (segment (start 102.87 157.48) (end 97.79 152.4) (width 0.25) (layer B.Cu) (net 15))
 (segment (start 105.41 157.48) (end 102.87 157.48) (width 0.25) (layer B.Cu) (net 15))
 (segment (start 114.3 168.91) (end 114.3 162.56) (width 0.25) (layer F.Cu) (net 34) (status 400000))
 (segment (start 114.3 162.56) (end 113.03 161.29) (width 0.25) (layer F.Cu) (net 34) (status 800000))
 (segment (start 40.64 139.7) (end 40.64 129.54) (width 0.25) (layer F.Cu) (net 30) (status C00000))
 (segment (start 40.64 129.54) (end 46.99 123.19) (width 0.25) (layer F.Cu) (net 30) (status 400000))
 (segment (start 46.99 123.19) (end 46.99 121.92) (width 0.25) (layer F.Cu) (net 30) (status 800000))
 (segment (start 86.36 111.18) (end 92.86 111.18) (width 0.25) (layer F.Cu) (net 33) (status C00000))
 (segment (start 81.28 118.11) (end 81.28 116.26) (width 0.25) (layer F.Cu) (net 33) (status 400000))
 (segment (start 81.28 116.26) (end 86.36 111.18) (width 0.25) (layer F.Cu) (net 33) (status 800000))
 (segment (start 81.28 133.35) (end 85.09 133.35) (width 0.25) (layer F.Cu) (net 20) (status 400000))
 (segment (start 87.63 134.62) (end 97.79 144.78) (width 0.25) (layer F.Cu) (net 20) (status 800000))
 (segment (start 86.36 134.62) (end 87.63 134.62) (width 0.25) (layer F.Cu) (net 20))
 (segment (start 85.09 133.35) (end 86.36 134.62) (width 0.25) (layer F.Cu) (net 20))
 (segment (start 73.66 111.18) (end 80.16 111.18) (width 0.25) (layer F.Cu) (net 32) (status C00000))
 (segment (start 72.39 118.11) (end 72.39 112.45) (width 0.25) (layer F.Cu) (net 32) (status 400000))
 (segment (start 72.39 112.45) (end 73.66 111.18) (width 0.25) (layer F.Cu) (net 32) (status 800000))
 (segment (start 97.79 147.32) (end 87.63 137.16) (width 0.25) (layer F.Cu) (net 18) (status 400000))
 (segment (start 76.2 137.16) (end 72.39 133.35) (width 0.25) (layer F.Cu) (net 18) (status 800000))
 (segment (start 87.63 137.16) (end 76.2 137.16) (width 0.25) (layer F.Cu) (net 18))
 (segment (start 67.31 111.33) (end 67.46 111.18) (width 0.25) (layer F.Cu) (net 31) (status C00000))
 (segment (start 67.31 111.33) (end 67.46 111.18) (width 0.25) (layer F.Cu) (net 31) (status C00000))
 (segment (start 67.46 111.18) (end 60.96 111.18) (width 0.25) (layer F.Cu) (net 31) (status C00000))
 (segment (start 63.5 118.11) (end 63.5 113.72) (width 0.25) (layer F.Cu) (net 31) (status 400000))
 (segment (start 63.5 113.72) (end 60.96 111.18) (width 0.25) (layer F.Cu) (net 31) (status 800000))
 (segment (start 63.5 133.35) (end 68.58 138.43) (width 0.25) (layer F.Cu) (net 16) (status 400000))
 (segment (start 86.36 138.43) (end 97.79 149.86) (width 0.25) (layer F.Cu) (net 16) (status 800000))
 (segment (start 85.09 138.43) (end 86.36 138.43) (width 0.25) (layer F.Cu) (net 16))
 (segment (start 68.58 138.43) (end 85.09 138.43) (width 0.25) (layer F.Cu) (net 16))
 (segment (start 98.91 111.76) (end 105.41 111.76) (width 0.25) (layer F.Cu) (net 26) (status C00000))
 (segment (start 97.79 137.16) (end 97.79 112.88) (width 0.25) (layer F.Cu) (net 26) (status 400000))
 (segment (start 97.79 112.88) (end 98.91 111.76) (width 0.25) (layer F.Cu) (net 26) (status 800000))
 (segment (start 105.41 137.16) (end 110.49 137.16) (width 0.25) (layer F.Cu) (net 1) (status C00000))
 (segment (start 110.49 137.16) (end 114.3 137.16) (width 0.25) (layer F.Cu) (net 1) (status 800000))
 (segment (start 105.41 139.7) (end 110.49 139.7) (width 0.25) (layer F.Cu) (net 3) (status C00000))
 (segment (start 110.49 139.7) (end 114.3 139.7) (width 0.25) (layer F.Cu) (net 3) (status 800000))
 (segment (start 87.63 127) (end 87.63 132.08) (width 0.25) (layer F.Cu) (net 22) (status 400000))
 (segment (start 87.63 132.08) (end 97.79 142.24) (width 0.25) (layer F.Cu) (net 22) (status 800000))
 (segment (start 97.79 139.7) (end 93.98 135.89) (width 0.25) (layer F.Cu) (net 24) (status 400000))
 (segment (start 93.98 125.73) (end 87.63 119.38) (width 0.25) (layer F.Cu) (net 24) (status 800000))
 (segment (start 93.98 135.89) (end 93.98 125.73) (width 0.25) (layer F.Cu) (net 24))
 (segment (start 104.284999 169.054999) (end 86.504999 169.054999) (width 0.25) (layer B.Cu) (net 25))
 (segment (start 105.41 170.18) (end 104.284999 169.054999) (width 0.25) (layer B.Cu) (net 25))
 (segment (start 86.504999 169.054999) (end 85.09 167.64) (width 0.25) (layer B.Cu) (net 25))
 (segment (start 85.09 124.46) (end 87.63 121.92) (width 0.25) (layer B.Cu) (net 25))
 (segment (start 85.09 167.64) (end 85.09 124.46) (width 0.25) (layer B.Cu) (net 25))
 (segment (start 97.539997 166.514999) (end 93.98 162.955002) (width 0.25) (layer B.Cu) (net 23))
 (segment (start 105.41 167.64) (end 104.284999 166.514999) (width 0.25) (layer B.Cu) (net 23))
 (segment (start 104.284999 166.514999) (end 97.539997 166.514999) (width 0.25) (layer B.Cu) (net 23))
 (segment (start 87.63 124.714998) (end 87.63 124.46) (width 0.25) (layer B.Cu) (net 23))
 (segment (start 93.98 131.064998) (end 87.63 124.714998) (width 0.25) (layer B.Cu) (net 23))
 (segment (start 93.98 162.955002) (end 93.98 131.064998) (width 0.25) (layer B.Cu) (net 23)))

